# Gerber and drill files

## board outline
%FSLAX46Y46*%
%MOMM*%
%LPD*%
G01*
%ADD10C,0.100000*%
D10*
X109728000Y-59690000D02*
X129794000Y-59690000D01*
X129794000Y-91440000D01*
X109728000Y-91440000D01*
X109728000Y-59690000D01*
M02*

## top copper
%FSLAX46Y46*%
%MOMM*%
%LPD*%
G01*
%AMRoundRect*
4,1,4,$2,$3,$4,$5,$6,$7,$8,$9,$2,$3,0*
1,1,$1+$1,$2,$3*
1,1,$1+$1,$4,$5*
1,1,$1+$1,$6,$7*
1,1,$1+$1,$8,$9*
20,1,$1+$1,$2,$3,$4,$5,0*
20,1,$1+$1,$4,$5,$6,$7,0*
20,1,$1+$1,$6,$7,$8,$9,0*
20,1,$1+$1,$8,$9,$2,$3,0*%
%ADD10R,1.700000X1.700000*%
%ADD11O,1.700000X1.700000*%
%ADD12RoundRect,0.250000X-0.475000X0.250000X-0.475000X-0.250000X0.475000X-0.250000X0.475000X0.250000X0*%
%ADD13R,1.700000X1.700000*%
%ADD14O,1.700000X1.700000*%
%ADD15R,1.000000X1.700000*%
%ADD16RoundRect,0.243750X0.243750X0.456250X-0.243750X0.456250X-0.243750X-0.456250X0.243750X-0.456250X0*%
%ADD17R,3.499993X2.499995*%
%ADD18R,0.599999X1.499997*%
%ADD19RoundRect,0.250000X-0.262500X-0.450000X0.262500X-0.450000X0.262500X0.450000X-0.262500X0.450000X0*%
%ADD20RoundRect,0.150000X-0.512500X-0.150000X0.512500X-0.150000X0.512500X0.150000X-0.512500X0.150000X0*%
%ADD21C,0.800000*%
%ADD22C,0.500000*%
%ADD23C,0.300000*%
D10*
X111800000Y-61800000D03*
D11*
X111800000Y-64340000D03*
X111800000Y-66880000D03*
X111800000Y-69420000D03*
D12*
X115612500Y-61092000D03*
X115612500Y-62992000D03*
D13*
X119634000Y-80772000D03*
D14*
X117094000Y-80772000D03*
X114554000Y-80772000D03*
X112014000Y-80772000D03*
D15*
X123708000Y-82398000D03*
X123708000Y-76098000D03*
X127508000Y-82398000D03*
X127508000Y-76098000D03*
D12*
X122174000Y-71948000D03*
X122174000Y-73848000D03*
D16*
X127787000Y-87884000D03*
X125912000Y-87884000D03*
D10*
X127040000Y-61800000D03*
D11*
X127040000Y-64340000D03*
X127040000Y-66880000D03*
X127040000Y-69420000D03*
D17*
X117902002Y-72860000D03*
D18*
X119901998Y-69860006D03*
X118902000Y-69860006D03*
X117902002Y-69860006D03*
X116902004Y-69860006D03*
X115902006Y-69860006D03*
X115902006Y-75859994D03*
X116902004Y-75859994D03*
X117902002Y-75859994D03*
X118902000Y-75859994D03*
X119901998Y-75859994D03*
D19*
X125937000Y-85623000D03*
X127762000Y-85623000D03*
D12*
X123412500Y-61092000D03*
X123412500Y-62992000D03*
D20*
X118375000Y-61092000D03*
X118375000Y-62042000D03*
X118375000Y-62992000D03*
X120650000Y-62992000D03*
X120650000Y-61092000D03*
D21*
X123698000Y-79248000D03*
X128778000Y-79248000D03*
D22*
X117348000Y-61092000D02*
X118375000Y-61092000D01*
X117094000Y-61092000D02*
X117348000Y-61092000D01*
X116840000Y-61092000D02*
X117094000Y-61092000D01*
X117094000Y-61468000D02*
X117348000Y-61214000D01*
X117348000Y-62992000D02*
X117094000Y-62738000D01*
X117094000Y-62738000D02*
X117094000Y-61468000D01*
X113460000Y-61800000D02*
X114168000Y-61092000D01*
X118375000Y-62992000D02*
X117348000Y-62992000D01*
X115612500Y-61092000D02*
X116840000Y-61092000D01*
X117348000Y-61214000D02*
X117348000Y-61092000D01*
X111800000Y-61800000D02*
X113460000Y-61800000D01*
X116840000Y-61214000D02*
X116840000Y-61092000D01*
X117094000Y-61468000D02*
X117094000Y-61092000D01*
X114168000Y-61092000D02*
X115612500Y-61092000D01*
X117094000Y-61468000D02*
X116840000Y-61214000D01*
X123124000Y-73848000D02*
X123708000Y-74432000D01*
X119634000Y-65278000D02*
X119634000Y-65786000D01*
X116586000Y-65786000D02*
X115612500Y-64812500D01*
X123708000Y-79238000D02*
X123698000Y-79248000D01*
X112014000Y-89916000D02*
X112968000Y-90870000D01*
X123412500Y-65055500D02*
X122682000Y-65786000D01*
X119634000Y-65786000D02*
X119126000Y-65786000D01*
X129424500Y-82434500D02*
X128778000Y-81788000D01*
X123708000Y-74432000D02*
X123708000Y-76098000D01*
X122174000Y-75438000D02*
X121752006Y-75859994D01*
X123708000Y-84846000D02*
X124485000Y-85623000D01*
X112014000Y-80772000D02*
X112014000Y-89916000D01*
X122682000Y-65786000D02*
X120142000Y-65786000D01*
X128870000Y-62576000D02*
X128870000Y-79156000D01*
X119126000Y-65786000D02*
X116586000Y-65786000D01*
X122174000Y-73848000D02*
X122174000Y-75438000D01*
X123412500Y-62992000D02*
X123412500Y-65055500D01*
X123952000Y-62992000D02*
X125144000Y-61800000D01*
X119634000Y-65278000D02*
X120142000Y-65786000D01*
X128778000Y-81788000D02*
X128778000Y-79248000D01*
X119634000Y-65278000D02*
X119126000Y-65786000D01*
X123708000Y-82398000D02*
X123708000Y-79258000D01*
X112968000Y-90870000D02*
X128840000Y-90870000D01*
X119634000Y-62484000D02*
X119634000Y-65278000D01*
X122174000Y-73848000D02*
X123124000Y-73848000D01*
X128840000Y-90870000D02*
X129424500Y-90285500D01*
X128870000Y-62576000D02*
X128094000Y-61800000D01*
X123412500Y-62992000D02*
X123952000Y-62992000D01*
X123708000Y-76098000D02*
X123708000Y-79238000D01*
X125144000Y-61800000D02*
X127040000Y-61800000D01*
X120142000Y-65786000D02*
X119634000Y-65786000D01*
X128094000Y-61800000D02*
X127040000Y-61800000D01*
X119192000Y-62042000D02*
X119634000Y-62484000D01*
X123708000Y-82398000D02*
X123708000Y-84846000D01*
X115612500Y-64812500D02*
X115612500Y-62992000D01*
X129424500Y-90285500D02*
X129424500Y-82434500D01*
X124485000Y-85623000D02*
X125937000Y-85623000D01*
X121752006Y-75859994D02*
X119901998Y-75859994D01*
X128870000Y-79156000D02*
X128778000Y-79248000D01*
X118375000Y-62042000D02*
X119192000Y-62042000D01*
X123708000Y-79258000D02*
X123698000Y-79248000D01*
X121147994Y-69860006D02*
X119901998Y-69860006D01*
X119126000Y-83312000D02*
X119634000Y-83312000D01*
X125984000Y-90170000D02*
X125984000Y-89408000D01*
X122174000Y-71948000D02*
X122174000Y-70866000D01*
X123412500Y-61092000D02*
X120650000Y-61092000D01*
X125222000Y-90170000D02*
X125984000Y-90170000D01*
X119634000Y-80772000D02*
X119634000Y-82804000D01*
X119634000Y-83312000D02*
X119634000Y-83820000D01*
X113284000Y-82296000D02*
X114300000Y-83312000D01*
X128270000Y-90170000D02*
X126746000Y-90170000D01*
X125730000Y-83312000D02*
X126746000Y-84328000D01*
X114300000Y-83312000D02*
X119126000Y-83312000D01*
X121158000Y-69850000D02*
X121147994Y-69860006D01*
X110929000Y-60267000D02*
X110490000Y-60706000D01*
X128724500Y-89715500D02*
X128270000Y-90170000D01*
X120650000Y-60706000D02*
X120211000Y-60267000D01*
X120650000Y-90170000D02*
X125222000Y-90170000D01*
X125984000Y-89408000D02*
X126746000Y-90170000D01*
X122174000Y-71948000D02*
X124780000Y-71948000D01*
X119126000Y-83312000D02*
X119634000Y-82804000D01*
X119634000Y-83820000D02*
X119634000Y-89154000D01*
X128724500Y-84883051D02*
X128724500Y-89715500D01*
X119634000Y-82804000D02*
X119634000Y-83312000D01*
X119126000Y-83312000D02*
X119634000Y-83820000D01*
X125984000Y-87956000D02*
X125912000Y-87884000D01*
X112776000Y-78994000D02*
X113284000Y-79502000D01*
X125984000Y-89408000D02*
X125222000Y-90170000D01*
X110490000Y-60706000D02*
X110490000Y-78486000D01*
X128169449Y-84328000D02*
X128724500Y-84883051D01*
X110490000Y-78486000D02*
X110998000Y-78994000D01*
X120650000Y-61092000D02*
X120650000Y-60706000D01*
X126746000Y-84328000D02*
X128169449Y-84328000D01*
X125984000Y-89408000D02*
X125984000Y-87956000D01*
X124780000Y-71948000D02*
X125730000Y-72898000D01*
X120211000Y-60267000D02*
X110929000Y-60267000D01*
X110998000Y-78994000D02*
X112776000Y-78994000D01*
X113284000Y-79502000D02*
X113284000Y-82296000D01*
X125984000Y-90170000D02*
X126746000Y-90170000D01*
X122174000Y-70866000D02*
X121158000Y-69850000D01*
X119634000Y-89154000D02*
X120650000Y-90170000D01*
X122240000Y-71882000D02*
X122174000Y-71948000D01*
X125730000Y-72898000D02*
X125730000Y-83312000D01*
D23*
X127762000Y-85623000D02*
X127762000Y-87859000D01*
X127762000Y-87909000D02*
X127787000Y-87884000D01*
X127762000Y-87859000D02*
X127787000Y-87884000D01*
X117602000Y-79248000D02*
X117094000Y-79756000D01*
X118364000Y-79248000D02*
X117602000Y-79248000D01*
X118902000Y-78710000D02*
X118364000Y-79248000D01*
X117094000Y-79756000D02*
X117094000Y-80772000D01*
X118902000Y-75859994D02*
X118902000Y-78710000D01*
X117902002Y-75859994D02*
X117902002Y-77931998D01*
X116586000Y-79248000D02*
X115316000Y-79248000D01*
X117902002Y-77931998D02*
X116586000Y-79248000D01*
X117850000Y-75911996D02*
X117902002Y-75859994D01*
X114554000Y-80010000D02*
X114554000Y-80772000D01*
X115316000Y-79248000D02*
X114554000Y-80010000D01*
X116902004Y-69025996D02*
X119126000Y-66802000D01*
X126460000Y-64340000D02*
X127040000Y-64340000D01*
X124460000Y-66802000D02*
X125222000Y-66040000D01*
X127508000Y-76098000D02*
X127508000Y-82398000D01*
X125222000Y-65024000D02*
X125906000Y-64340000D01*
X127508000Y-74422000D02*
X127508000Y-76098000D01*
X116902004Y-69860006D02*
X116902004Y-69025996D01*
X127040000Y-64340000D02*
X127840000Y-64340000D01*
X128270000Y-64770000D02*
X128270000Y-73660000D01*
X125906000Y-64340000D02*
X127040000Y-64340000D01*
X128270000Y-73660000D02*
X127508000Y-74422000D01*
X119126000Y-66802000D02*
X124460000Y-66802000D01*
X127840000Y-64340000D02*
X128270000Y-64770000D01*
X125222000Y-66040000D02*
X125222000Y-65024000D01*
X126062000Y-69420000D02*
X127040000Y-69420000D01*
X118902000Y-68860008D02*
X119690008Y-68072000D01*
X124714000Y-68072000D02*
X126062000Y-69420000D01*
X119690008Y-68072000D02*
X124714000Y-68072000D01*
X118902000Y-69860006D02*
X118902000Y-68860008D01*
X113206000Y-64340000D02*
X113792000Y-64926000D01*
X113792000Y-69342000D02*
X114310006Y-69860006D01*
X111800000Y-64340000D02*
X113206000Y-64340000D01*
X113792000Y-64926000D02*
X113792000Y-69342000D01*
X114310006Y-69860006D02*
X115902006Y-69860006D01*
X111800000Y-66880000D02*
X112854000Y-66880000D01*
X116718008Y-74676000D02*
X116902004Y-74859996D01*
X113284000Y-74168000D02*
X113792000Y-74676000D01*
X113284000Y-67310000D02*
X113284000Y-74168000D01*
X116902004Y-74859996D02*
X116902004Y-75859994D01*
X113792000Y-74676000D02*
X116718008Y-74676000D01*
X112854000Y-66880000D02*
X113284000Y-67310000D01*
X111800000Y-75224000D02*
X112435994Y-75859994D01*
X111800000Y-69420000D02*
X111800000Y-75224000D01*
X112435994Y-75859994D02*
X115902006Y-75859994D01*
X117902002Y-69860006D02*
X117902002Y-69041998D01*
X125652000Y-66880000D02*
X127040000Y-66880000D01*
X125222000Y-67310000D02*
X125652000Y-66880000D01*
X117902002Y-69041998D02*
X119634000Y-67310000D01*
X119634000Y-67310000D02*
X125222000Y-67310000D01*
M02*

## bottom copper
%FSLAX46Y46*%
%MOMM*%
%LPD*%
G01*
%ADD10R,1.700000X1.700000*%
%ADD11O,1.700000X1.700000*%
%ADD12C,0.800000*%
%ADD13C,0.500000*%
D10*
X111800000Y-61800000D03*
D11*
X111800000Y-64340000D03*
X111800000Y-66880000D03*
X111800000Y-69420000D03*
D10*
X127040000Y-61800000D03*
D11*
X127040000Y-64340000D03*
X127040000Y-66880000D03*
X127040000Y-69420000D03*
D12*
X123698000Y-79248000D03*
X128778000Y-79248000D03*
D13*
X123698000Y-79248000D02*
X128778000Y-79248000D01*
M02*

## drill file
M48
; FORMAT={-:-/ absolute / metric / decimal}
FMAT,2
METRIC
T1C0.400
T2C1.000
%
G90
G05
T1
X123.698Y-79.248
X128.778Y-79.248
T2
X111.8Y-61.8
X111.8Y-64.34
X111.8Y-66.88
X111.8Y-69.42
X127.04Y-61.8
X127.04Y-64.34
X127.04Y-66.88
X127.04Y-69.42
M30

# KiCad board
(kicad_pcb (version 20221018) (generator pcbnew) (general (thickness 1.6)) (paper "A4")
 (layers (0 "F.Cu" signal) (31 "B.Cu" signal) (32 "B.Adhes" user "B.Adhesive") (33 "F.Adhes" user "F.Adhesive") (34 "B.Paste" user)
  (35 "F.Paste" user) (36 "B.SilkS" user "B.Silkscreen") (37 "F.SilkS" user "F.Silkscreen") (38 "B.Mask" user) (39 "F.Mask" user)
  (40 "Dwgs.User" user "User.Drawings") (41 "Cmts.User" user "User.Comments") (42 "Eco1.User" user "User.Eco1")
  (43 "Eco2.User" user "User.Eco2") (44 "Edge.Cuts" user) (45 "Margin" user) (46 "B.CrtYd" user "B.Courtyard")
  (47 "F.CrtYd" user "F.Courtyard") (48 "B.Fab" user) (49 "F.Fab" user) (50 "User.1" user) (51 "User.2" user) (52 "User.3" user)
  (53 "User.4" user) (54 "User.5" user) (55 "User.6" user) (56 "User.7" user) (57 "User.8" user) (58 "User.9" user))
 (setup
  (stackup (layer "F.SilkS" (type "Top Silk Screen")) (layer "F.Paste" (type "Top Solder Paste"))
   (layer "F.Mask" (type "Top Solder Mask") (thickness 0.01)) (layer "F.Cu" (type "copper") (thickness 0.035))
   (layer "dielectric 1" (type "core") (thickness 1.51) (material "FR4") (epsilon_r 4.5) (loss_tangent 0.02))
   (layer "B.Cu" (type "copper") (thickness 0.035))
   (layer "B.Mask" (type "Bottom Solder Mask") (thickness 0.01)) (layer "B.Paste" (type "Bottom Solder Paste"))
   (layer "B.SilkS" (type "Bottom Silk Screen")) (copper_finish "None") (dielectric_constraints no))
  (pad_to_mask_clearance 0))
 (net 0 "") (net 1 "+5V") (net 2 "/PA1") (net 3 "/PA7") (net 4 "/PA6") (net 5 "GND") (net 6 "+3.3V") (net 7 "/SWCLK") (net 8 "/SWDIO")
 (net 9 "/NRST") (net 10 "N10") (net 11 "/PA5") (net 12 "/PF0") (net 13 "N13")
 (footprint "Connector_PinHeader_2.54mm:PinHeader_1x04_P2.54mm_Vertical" (layer "F.Cu") (at 111.8 61.8)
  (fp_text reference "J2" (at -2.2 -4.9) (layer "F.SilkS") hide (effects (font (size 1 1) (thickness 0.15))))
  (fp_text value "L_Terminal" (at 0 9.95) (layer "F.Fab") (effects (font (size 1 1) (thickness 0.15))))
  (pad "1" thru_hole rect (at 0 0) (size 1.7 1.7) (drill 1) (layers "*.Cu" "*.Mask") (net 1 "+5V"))
  (pad "2" thru_hole oval (at 0 2.54) (size 1.7 1.7) (drill 1) (layers "*.Cu" "*.Mask") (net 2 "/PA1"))
  (pad "3" thru_hole oval (at 0 5.08) (size 1.7 1.7) (drill 1) (layers "*.Cu" "*.Mask") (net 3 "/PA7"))
  (pad "4" thru_hole oval (at 0 7.62) (size 1.7 1.7) (drill 1) (layers "*.Cu" "*.Mask") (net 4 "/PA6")))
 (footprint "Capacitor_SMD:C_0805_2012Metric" (layer "F.Cu") (at 115.6125 62.042 -90)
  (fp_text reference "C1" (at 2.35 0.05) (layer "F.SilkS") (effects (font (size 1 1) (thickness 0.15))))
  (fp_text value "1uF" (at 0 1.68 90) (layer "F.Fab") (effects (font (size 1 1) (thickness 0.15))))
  (pad "1" smd roundrect (at -0.95 0 270) (size 1 1.45) (layers "F.Cu" "F.Paste" "F.Mask") (roundrect_rratio 0.25) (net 1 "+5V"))
  (pad "2" smd roundrect (at 0.95 0 270) (size 1 1.45) (layers "F.Cu" "F.Paste" "F.Mask") (roundrect_rratio 0.25) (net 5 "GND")))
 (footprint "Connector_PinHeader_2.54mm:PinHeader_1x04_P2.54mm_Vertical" (layer "F.Cu") (at 119.634 80.772 -90)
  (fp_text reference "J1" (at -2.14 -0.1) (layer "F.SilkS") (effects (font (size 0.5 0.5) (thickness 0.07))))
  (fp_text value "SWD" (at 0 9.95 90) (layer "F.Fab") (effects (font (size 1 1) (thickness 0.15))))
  (pad "1" smd rect (at 0 0 270) (size 1.7 1.7) (layers "F.Cu" "F.Paste" "F.Mask") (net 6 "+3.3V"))
  (pad "2" smd oval (at 0 2.54 270) (size 1.7 1.7) (layers "F.Cu" "F.Paste" "F.Mask") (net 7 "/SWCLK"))
  (pad "3" smd oval (at 0 5.08 270) (size 1.7 1.7) (layers "F.Cu" "F.Paste" "F.Mask") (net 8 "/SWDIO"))
  (pad "4" smd oval (at 0 7.62 270) (size 1.7 1.7) (layers "F.Cu" "F.Paste" "F.Mask") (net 5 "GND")))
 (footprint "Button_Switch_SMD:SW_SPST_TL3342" (layer "F.Cu") (at 125.608 79.248 90)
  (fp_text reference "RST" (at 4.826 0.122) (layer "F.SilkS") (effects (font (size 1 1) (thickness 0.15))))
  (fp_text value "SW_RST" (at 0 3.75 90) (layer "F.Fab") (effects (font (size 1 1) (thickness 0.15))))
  (pad "1" smd rect (at -3.15 -1.9 90) (size 1.7 1) (layers "F.Cu" "F.Paste" "F.Mask") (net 5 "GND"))
  (pad "1" smd rect (at 3.15 -1.9 90) (size 1.7 1) (layers "F.Cu" "F.Paste" "F.Mask") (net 5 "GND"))
  (pad "2" smd rect (at -3.15 1.9 90) (size 1.7 1) (layers "F.Cu" "F.Paste" "F.Mask") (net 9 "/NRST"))
  (pad "2" smd rect (at 3.15 1.9 90) (size 1.7 1) (layers "F.Cu" "F.Paste" "F.Mask") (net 9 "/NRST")))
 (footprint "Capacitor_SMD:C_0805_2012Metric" (layer "F.Cu") (at 122.174 72.898 -90)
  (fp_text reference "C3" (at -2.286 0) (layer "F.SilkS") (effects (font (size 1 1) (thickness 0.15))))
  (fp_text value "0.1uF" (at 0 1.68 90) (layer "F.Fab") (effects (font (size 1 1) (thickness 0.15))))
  (pad "1" smd roundrect (at -0.95 0 270) (size 1 1.45) (layers "F.Cu" "F.Paste" "F.Mask") (roundrect_rratio 0.25) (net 6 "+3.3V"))
  (pad "2" smd roundrect (at 0.95 0 270) (size 1 1.45) (layers "F.Cu" "F.Paste" "F.Mask") (roundrect_rratio 0.25) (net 5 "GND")))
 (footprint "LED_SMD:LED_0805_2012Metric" (layer "F.Cu") (at 126.8495 87.884 180)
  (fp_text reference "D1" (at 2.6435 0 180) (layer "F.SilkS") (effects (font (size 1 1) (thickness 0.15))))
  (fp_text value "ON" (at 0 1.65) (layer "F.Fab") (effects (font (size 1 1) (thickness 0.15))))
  (pad "1" smd roundrect (at -0.9375 0 180) (size 0.975 1.4) (layers "F.Cu" "F.Paste" "F.Mask") (roundrect_rratio 0.25) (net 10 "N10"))
  (pad "2" smd roundrect (at 0.9375 0 180) (size 0.975 1.4) (layers "F.Cu" "F.Paste" "F.Mask") (roundrect_rratio 0.25) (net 6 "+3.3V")))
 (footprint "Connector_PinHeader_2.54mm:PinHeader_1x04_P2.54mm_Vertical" (layer "F.Cu") (at 127.04 61.8)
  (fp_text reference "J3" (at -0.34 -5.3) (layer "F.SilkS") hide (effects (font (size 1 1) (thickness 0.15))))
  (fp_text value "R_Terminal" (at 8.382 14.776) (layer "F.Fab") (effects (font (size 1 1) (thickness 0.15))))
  (pad "1" thru_hole rect (at 0 0) (size 1.7 1.7) (drill 1) (layers "*.Cu" "*.Mask") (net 5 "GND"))
  (pad "2" thru_hole oval (at 0 2.54) (size 1.7 1.7) (drill 1) (layers "*.Cu" "*.Mask") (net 9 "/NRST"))
  (pad "3" thru_hole oval (at 0 5.08) (size 1.7 1.7) (drill 1) (layers "*.Cu" "*.Mask") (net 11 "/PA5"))
  (pad "4" thru_hole oval (at 0 7.62) (size 1.7 1.7) (drill 1) (layers "*.Cu" "*.Mask") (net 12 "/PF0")))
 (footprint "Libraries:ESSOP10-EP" (layer "F.Cu") (at 117.902002 72.859873 -90)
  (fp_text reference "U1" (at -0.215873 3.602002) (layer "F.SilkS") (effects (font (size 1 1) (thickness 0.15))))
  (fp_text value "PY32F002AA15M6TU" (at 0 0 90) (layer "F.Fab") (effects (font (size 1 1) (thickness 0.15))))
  (pad "0" smd rect (at 0.000127 0 270) (size 2.499995 3.499993) (layers "F.Cu" "F.Paste" "F.Mask"))
  (pad "1" smd rect (at -2.999867 -1.999996 270) (size 1.499997 0.599999) (layers "F.Cu" "F.Paste" "F.Mask") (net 6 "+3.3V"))
  (pad "2" smd rect (at -2.999867 -0.999998 270) (size 1.499997 0.599999) (layers "F.Cu" "F.Paste" "F.Mask") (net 12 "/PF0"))
  (pad "3" smd rect (at -2.999867 0 270) (size 1.499997 0.599999) (layers "F.Cu" "F.Paste" "F.Mask") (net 11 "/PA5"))
  (pad "4" smd rect (at -2.999867 0.999998 270) (size 1.499997 0.599999) (layers "F.Cu" "F.Paste" "F.Mask") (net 9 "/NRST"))
  (pad "5" smd rect (at -2.999867 1.999996 270) (size 1.499997 0.599999) (layers "F.Cu" "F.Paste" "F.Mask") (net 2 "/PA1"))
  (pad "6" smd rect (at 3.000121 1.999996 270) (size 1.499997 0.599999) (layers "F.Cu" "F.Paste" "F.Mask") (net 4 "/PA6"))
  (pad "7" smd rect (at 3.000121 0.999998 270) (size 1.499997 0.599999) (layers "F.Cu" "F.Paste" "F.Mask") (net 3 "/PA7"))
  (pad "8" smd rect (at 3.000121 0 270) (size 1.499997 0.599999) (layers "F.Cu" "F.Paste" "F.Mask") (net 8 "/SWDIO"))
  (pad "9" smd rect (at 3.000121 -0.999998 270) (size 1.499997 0.599999) (layers "F.Cu" "F.Paste" "F.Mask") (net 7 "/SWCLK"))
  (pad "10" smd rect (at 3.000121 -1.999996 270) (size 1.499997 0.599999) (layers "F.Cu" "F.Paste" "F.Mask") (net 5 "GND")))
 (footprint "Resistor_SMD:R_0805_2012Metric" (layer "F.Cu") (at 126.8495 85.623)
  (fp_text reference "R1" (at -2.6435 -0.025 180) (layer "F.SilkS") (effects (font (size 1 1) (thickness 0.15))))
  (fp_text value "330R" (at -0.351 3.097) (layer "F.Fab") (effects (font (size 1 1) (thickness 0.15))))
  (pad "1" smd roundrect (at -0.9125 0) (size 1.025 1.4) (layers "F.Cu" "F.Paste" "F.Mask") (roundrect_rratio 0.243902) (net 5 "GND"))
  (pad "2" smd roundrect (at 0.9125 0) (size 1.025 1.4) (layers "F.Cu" "F.Paste" "F.Mask") (roundrect_rratio 0.243902) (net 10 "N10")))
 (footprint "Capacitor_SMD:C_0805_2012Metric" (layer "F.Cu") (at 123.4125 62.042 -90)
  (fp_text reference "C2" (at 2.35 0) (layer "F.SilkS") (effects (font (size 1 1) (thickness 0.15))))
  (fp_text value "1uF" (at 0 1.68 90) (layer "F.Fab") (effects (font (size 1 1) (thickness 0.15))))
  (pad "1" smd roundrect (at -0.95 0 270) (size 1 1.45) (layers "F.Cu" "F.Paste" "F.Mask") (roundrect_rratio 0.25) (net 6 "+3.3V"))
  (pad "2" smd roundrect (at 0.95 0 270) (size 1 1.45) (layers "F.Cu" "F.Paste" "F.Mask") (roundrect_rratio 0.25) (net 5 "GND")))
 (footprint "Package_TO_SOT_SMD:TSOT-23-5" (layer "F.Cu") (at 119.5125 62.042)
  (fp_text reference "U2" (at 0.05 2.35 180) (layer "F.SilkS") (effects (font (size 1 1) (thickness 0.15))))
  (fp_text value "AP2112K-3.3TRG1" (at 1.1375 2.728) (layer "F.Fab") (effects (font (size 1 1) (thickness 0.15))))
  (pad "1" smd roundrect (at -1.1375 -0.95) (size 1.325 0.6) (layers "F.Cu" "F.Paste" "F.Mask") (roundrect_rratio 0.25) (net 1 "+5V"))
  (pad "2" smd roundrect (at -1.1375 0) (size 1.325 0.6) (layers "F.Cu" "F.Paste" "F.Mask") (roundrect_rratio 0.25) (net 5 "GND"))
  (pad "3" smd roundrect (at -1.1375 0.95) (size 1.325 0.6) (layers "F.Cu" "F.Paste" "F.Mask") (roundrect_rratio 0.25) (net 1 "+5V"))
  (pad "4" smd roundrect (at 1.1375 0.95) (size 1.325 0.6) (layers "F.Cu" "F.Paste" "F.Mask") (roundrect_rratio 0.25) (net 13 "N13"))
  (pad "5" smd roundrect (at 1.1375 -0.95) (size 1.325 0.6) (layers "F.Cu" "F.Paste" "F.Mask") (roundrect_rratio 0.25) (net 6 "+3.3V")))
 (gr_rect (start 109.728 59.69) (end 129.794 91.44) (stroke (width 0.1) (type default)) (fill none) (layer "Edge.Cuts"))
 (segment (start 117.348 61.092) (end 118.375 61.092) (width 0.5) (layer "F.Cu") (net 1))
 (segment (start 117.094 61.092) (end 117.348 61.092) (width 0.5) (layer "F.Cu") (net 1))
 (segment (start 116.84 61.092) (end 117.094 61.092) (width 0.5) (layer "F.Cu") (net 1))
 (segment (start 117.094 61.468) (end 117.348 61.214) (width 0.5) (layer "F.Cu") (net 1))
 (segment (start 117.348 62.992) (end 117.094 62.738) (width 0.5) (layer "F.Cu") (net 1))
 (segment (start 117.094 62.738) (end 117.094 61.468) (width 0.5) (layer "F.Cu") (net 1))
 (segment (start 113.46 61.8) (end 114.168 61.092) (width 0.5) (layer "F.Cu") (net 1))
 (segment (start 118.375 62.992) (end 117.348 62.992) (width 0.5) (layer "F.Cu") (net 1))
 (segment (start 115.6125 61.092) (end 116.84 61.092) (width 0.5) (layer "F.Cu") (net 1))
 (segment (start 117.348 61.214) (end 117.348 61.092) (width 0.5) (layer "F.Cu") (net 1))
 (segment (start 111.8 61.8) (end 113.46 61.8) (width 0.5) (layer "F.Cu") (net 1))
 (segment (start 116.84 61.214) (end 116.84 61.092) (width 0.5) (layer "F.Cu") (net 1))
 (segment (start 117.094 61.468) (end 117.094 61.092) (width 0.5) (layer "F.Cu") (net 1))
 (segment (start 114.168 61.092) (end 115.6125 61.092) (width 0.5) (layer "F.Cu") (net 1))
 (segment (start 117.094 61.468) (end 116.84 61.214) (width 0.5) (layer "F.Cu") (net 1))
 (segment (start 123.124 73.848) (end 123.708 74.432) (width 0.5) (layer "F.Cu") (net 5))
 (segment (start 119.634 65.278) (end 119.634 65.786) (width 0.5) (layer "F.Cu") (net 5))
 (segment (start 116.586 65.786) (end 115.6125 64.8125) (width 0.5) (layer "F.Cu") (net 5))
 (segment (start 123.708 79.238) (end 123.698 79.248) (width 0.5) (layer "F.Cu") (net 5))
 (segment (start 112.014 89.916) (end 112.968 90.87) (width 0.5) (layer "F.Cu") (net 5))
 (segment (start 123.4125 65.0555) (end 122.682 65.786) (width 0.5) (layer "F.Cu") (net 5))
 (segment (start 119.634 65.786) (end 119.126 65.786) (width 0.5) (layer "F.Cu") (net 5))
 (segment (start 129.4245 82.4345) (end 128.778 81.788) (width 0.5) (layer "F.Cu") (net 5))
 (segment (start 123.708 74.432) (end 123.708 76.098) (width 0.5) (layer "F.Cu") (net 5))
 (segment (start 122.174 75.438) (end 121.752006 75.859994) (width 0.5) (layer "F.Cu") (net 5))
 (segment (start 123.708 84.846) (end 124.485 85.623) (width 0.5) (layer "F.Cu") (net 5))
 (segment (start 112.014 80.772) (end 112.014 89.916) (width 0.5) (layer "F.Cu") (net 5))
 (segment (start 122.682 65.786) (end 120.142 65.786) (width 0.5) (layer "F.Cu") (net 5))
 (segment (start 128.87 62.576) (end 128.87 79.156) (width 0.5) (layer "F.Cu") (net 5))
 (segment (start 119.126 65.786) (end 116.586 65.786) (width 0.5) (layer "F.Cu") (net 5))
 (segment (start 122.174 73.848) (end 122.174 75.438) (width 0.5) (layer "F.Cu") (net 5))
 (segment (start 123.4125 62.992) (end 123.4125 65.0555) (width 0.5) (layer "F.Cu") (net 5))
 (segment (start 123.952 62.992) (end 125.144 61.8) (width 0.5) (layer "F.Cu") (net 5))
 (segment (start 119.634 65.278) (end 120.142 65.786) (width 0.5) (layer "F.Cu") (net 5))
 (segment (start 128.778 81.788) (end 128.778 79.248) (width 0.5) (layer "F.Cu") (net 5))
 (segment (start 119.634 65.278) (end 119.126 65.786) (width 0.5) (layer "F.Cu") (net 5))
 (segment (start 123.708 82.398) (end 123.708 79.258) (width 0.5) (layer "F.Cu") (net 5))
 (segment (start 112.968 90.87) (end 128.84 90.87) (width 0.5) (layer "F.Cu") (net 5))
 (segment (start 119.634 62.484) (end 119.634 65.278) (width 0.5) (layer "F.Cu") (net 5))
 (segment (start 122.174 73.848) (end 123.124 73.848) (width 0.5) (layer "F.Cu") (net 5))
 (segment (start 128.84 90.87) (end 129.4245 90.2855) (width 0.5) (layer "F.Cu") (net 5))
 (segment (start 128.87 62.576) (end 128.094 61.8) (width 0.5) (layer "F.Cu") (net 5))
 (segment (start 123.4125 62.992) (end 123.952 62.992) (width 0.5) (layer "F.Cu") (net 5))
 (segment (start 123.708 76.098) (end 123.708 79.238) (width 0.5) (layer "F.Cu") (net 5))
 (segment (start 125.144 61.8) (end 127.04 61.8) (width 0.5) (layer "F.Cu") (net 5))
 (segment (start 120.142 65.786) (end 119.634 65.786) (width 0.5) (layer "F.Cu") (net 5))
 (segment (start 128.094 61.8) (end 127.04 61.8) (width 0.5) (layer "F.Cu") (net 5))
 (segment (start 119.192 62.042) (end 119.634 62.484) (width 0.5) (layer "F.Cu") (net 5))
 (segment (start 123.708 82.398) (end 123.708 84.846) (width 0.5) (layer "F.Cu") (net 5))
 (segment (start 115.6125 64.8125) (end 115.6125 62.992) (width 0.5) (layer "F.Cu") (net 5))
 (segment (start 129.4245 90.2855) (end 129.4245 82.4345) (width 0.5) (layer "F.Cu") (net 5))
 (segment (start 124.485 85.623) (end 125.937 85.623) (width 0.5) (layer "F.Cu") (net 5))
 (segment (start 121.752006 75.859994) (end 119.901998 75.859994) (width 0.5) (layer "F.Cu") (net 5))
 (segment (start 128.87 79.156) (end 128.778 79.248) (width 0.5) (layer "F.Cu") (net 5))
 (segment (start 118.375 62.042) (end 119.192 62.042) (width 0.5) (layer "F.Cu") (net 5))
 (segment (start 123.708 79.258) (end 123.698 79.248) (width 0.5) (layer "F.Cu") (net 5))
 (via (at 123.698 79.248) (size 0.8) (drill 0.4) (layers "F.Cu" "B.Cu") (free) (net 5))
 (via (at 128.778 79.248) (size 0.8) (drill 0.4) (layers "F.Cu" "B.Cu") (free) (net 5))
 (segment (start 123.698 79.248) (end 128.778 79.248) (width 0.5) (layer "B.Cu") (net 5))
 (segment (start 121.147994 69.860006) (end 119.901998 69.860006) (width 0.5) (layer "F.Cu") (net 6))
 (segment (start 119.126 83.312) (end 119.634 83.312) (width 0.5) (layer "F.Cu") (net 6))
 (segment (start 125.984 90.17) (end 125.984 89.408) (width 0.5) (layer "F.Cu") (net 6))
 (segment (start 122.174 71.948) (end 122.174 70.866) (width 0.5) (layer "F.Cu") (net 6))
 (segment (start 123.4125 61.092) (end 120.65 61.092) (width 0.5) (layer "F.Cu") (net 6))
 (segment (start 125.222 90.17) (end 125.984 90.17) (width 0.5) (layer "F.Cu") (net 6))
 (segment (start 119.634 80.772) (end 119.634 82.804) (width 0.5) (layer "F.Cu") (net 6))
 (segment (start 119.634 83.312) (end 119.634 83.82) (width 0.5) (layer "F.Cu") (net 6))
 (segment (start 113.284 82.296) (end 114.3 83.312) (width 0.5) (layer "F.Cu") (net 6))
 (segment (start 128.27 90.17) (end 126.746 90.17) (width 0.5) (layer "F.Cu") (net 6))
 (segment (start 125.73 83.312) (end 126.746 84.328) (width 0.5) (layer "F.Cu") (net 6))
 (segment (start 114.3 83.312) (end 119.126 83.312) (width 0.5) (layer "F.Cu") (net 6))
 (segment (start 121.158 69.85) (end 121.147994 69.860006) (width 0.5) (layer "F.Cu") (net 6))
 (segment (start 110.929 60.267) (end 110.49 60.706) (width 0.5) (layer "F.Cu") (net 6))
 (segment (start 128.7245 89.7155) (end 128.27 90.17) (width 0.5) (layer "F.Cu") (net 6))
 (segment (start 120.65 60.706) (end 120.211 60.267) (width 0.5) (layer "F.Cu") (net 6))
 (segment (start 120.65 90.17) (end 125.222 90.17) (width 0.5) (layer "F.Cu") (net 6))
 (segment (start 125.984 89.408) (end 126.746 90.17) (width 0.5) (layer "F.Cu") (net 6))
 (segment (start 122.174 71.948) (end 124.78 71.948) (width 0.5) (layer "F.Cu") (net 6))
 (segment (start 119.126 83.312) (end 119.634 82.804) (width 0.5) (layer "F.Cu") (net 6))
 (segment (start 119.634 83.82) (end 119.634 89.154) (width 0.5) (layer "F.Cu") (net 6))
 (segment (start 128.7245 84.883051) (end 128.7245 89.7155) (width 0.5) (layer "F.Cu") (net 6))
 (segment (start 119.634 82.804) (end 119.634 83.312) (width 0.5) (layer "F.Cu") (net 6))
 (segment (start 119.126 83.312) (end 119.634 83.82) (width 0.5) (layer "F.Cu") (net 6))
 (segment (start 125.984 87.956) (end 125.912 87.884) (width 0.5) (layer "F.Cu") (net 6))
 (segment (start 112.776 78.994) (end 113.284 79.502) (width 0.5) (layer "F.Cu") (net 6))
 (segment (start 125.984 89.408) (end 125.222 90.17) (width 0.5) (layer "F.Cu") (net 6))
 (segment (start 110.49 60.706) (end 110.49 78.486) (width 0.5) (layer "F.Cu") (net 6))
 (segment (start 128.169449 84.328) (end 128.7245 84.883051) (width 0.5) (layer "F.Cu") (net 6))
 (segment (start 110.49 78.486) (end 110.998 78.994) (width 0.5) (layer "F.Cu") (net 6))
 (segment (start 120.65 61.092) (end 120.65 60.706) (width 0.5) (layer "F.Cu") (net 6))
 (segment (start 126.746 84.328) (end 128.169449 84.328) (width 0.5) (layer "F.Cu") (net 6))
 (segment (start 125.984 89.408) (end 125.984 87.956) (width 0.5) (layer "F.Cu") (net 6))
 (segment (start 124.78 71.948) (end 125.73 72.898) (width 0.5) (layer "F.Cu") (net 6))
 (segment (start 120.211 60.267) (end 110.929 60.267) (width 0.5) (layer "F.Cu") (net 6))
 (segment (start 110.998 78.994) (end 112.776 78.994) (width 0.5) (layer "F.Cu") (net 6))
 (segment (start 113.284 79.502) (end 113.284 82.296) (width 0.5) (layer "F.Cu") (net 6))
 (segment (start 125.984 90.17) (end 126.746 90.17) (width 0.5) (layer "F.Cu") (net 6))
 (segment (start 122.174 70.866) (end 121.158 69.85) (width 0.5) (layer "F.Cu") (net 6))
 (segment (start 119.634 89.154) (end 120.65 90.17) (width 0.5) (layer "F.Cu") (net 6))
 (segment (start 122.24 71.882) (end 122.174 71.948) (width 0.5) (layer "F.Cu") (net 6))
 (segment (start 125.73 72.898) (end 125.73 83.312) (width 0.5) (layer "F.Cu") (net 6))
 (segment (start 127.762 85.623) (end 127.762 87.859) (width 0.3) (layer "F.Cu") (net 10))
 (segment (start 127.762 87.909) (end 127.787 87.884) (width 0.3) (layer "F.Cu") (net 10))
 (segment (start 127.762 87.859) (end 127.787 87.884) (width 0.3) (layer "F.Cu") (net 10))
 (segment (start 117.602 79.248) (end 117.094 79.756) (width 0.3) (layer "F.Cu") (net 7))
 (segment (start 118.364 79.248) (end 117.602 79.248) (width 0.3) (layer "F.Cu") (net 7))
 (segment (start 118.902 78.71) (end 118.364 79.248) (width 0.3) (layer "F.Cu") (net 7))
 (segment (start 117.094 79.756) (end 117.094 80.772) (width 0.3) (layer "F.Cu") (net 7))
 (segment (start 118.902 75.859994) (end 118.902 78.71) (width 0.3) (layer "F.Cu") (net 7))
 (segment (start 117.902002 75.859994) (end 117.902002 77.931998) (width 0.3) (layer "F.Cu") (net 8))
 (segment (start 116.586 79.248) (end 115.316 79.248) (width 0.3) (layer "F.Cu") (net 8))
 (segment (start 117.902002 77.931998) (end 116.586 79.248) (width 0.3) (layer "F.Cu") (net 8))
 (segment (start 117.85 75.911996) (end 117.902002 75.859994) (width 0.3) (layer "F.Cu") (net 8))
 (segment (start 114.554 80.01) (end 114.554 80.772) (width 0.3) (layer "F.Cu") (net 8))
 (segment (start 115.316 79.248) (end 114.554 80.01) (width 0.3) (layer "F.Cu") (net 8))
 (segment (start 116.902004 69.025996) (end 119.126 66.802) (width 0.3) (layer "F.Cu") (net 9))
 (segment (start 126.46 64.34) (end 127.04 64.34) (width 0.3) (layer "F.Cu") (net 9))
 (segment (start 124.46 66.802) (end 125.222 66.04) (width 0.3) (layer "F.Cu") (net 9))
 (segment (start 127.508 76.098) (end 127.508 82.398) (width 0.3) (layer "F.Cu") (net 9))
 (segment (start 125.222 65.024) (end 125.906 64.34) (width 0.3) (layer "F.Cu") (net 9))
 (segment (start 127.508 74.422) (end 127.508 76.098) (width 0.3) (layer "F.Cu") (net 9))
 (segment (start 116.902004 69.860006) (end 116.902004 69.025996) (width 0.3) (layer "F.Cu") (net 9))
 (segment (start 127.04 64.34) (end 127.84 64.34) (width 0.3) (layer "F.Cu") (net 9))
 (segment (start 128.27 64.77) (end 128.27 73.66) (width 0.3) (layer "F.Cu") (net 9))
 (segment (start 125.906 64.34) (end 127.04 64.34) (width 0.3) (layer "F.Cu") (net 9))
 (segment (start 128.27 73.66) (end 127.508 74.422) (width 0.3) (layer "F.Cu") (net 9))
 (segment (start 119.126 66.802) (end 124.46 66.802) (width 0.3) (layer "F.Cu") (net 9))
 (segment (start 127.84 64.34) (end 128.27 64.77) (width 0.3) (layer "F.Cu") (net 9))
 (segment (start 125.222 66.04) (end 125.222 65.024) (width 0.3) (layer "F.Cu") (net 9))
 (segment (start 126.062 69.42) (end 127.04 69.42) (width 0.3) (layer "F.Cu") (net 12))
 (segment (start 118.902 68.860008) (end 119.690008 68.072) (width 0.3) (layer "F.Cu") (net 12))
 (segment (start 124.714 68.072) (end 126.062 69.42) (width 0.3) (layer "F.Cu") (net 12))
 (segment (start 119.690008 68.072) (end 124.714 68.072) (width 0.3) (layer "F.Cu") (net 12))
 (segment (start 118.902 69.860006) (end 118.902 68.860008) (width 0.3) (layer "F.Cu") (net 12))
 (segment (start 113.206 64.34) (end 113.792 64.926) (width 0.3) (layer "F.Cu") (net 2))
 (segment (start 113.792 69.342) (end 114.310006 69.860006) (width 0.3) (layer "F.Cu") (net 2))
 (segment (start 111.8 64.34) (end 113.206 64.34) (width 0.3) (layer "F.Cu") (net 2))
 (segment (start 113.792 64.926) (end 113.792 69.342) (width 0.3) (layer "F.Cu") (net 2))
 (segment (start 114.310006 69.860006) (end 115.902006 69.860006) (width 0.3) (layer "F.Cu") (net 2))
 (segment (start 111.8 66.88) (end 112.854 66.88) (width 0.3) (layer "F.Cu") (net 3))
 (segment (start 116.718008 74.676) (end 116.902004 74.859996) (width 0.3) (layer "F.Cu") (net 3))
 (segment (start 113.284 74.168) (end 113.792 74.676) (width 0.3) (layer "F.Cu") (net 3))
 (segment (start 113.284 67.31) (end 113.284 74.168) (width 0.3) (layer "F.Cu") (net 3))
 (segment (start 116.902004 74.859996) (end 116.902004 75.859994) (width 0.3) (layer "F.Cu") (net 3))
 (segment (start 113.792 74.676) (end 116.718008 74.676) (width 0.3) (layer "F.Cu") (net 3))
 (segment (start 112.854 66.88) (end 113.284 67.31) (width 0.3) (layer "F.Cu") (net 3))
 (segment (start 111.8 75.224) (end 112.435994 75.859994) (width 0.3) (layer "F.Cu") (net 4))
 (segment (start 111.8 69.42) (end 111.8 75.224) (width 0.3) (layer "F.Cu") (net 4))
 (segment (start 112.435994 75.859994) (end 115.902006 75.859994) (width 0.3) (layer "F.Cu") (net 4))
 (segment (start 117.902002 69.860006) (end 117.902002 69.041998) (width 0.3) (layer "F.Cu") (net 11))
 (segment (start 125.652 66.88) (end 127.04 66.88) (width 0.3) (layer "F.Cu") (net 11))
 (segment (start 125.222 67.31) (end 125.652 66.88) (width 0.3) (layer "F.Cu") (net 11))
 (segment (start 117.902002 69.041998) (end 119.634 67.31) (width 0.3) (layer "F.Cu") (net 11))
 (segment (start 119.634 67.31) (end 125.222 67.31) (width 0.3) (layer "F.Cu") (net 11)))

